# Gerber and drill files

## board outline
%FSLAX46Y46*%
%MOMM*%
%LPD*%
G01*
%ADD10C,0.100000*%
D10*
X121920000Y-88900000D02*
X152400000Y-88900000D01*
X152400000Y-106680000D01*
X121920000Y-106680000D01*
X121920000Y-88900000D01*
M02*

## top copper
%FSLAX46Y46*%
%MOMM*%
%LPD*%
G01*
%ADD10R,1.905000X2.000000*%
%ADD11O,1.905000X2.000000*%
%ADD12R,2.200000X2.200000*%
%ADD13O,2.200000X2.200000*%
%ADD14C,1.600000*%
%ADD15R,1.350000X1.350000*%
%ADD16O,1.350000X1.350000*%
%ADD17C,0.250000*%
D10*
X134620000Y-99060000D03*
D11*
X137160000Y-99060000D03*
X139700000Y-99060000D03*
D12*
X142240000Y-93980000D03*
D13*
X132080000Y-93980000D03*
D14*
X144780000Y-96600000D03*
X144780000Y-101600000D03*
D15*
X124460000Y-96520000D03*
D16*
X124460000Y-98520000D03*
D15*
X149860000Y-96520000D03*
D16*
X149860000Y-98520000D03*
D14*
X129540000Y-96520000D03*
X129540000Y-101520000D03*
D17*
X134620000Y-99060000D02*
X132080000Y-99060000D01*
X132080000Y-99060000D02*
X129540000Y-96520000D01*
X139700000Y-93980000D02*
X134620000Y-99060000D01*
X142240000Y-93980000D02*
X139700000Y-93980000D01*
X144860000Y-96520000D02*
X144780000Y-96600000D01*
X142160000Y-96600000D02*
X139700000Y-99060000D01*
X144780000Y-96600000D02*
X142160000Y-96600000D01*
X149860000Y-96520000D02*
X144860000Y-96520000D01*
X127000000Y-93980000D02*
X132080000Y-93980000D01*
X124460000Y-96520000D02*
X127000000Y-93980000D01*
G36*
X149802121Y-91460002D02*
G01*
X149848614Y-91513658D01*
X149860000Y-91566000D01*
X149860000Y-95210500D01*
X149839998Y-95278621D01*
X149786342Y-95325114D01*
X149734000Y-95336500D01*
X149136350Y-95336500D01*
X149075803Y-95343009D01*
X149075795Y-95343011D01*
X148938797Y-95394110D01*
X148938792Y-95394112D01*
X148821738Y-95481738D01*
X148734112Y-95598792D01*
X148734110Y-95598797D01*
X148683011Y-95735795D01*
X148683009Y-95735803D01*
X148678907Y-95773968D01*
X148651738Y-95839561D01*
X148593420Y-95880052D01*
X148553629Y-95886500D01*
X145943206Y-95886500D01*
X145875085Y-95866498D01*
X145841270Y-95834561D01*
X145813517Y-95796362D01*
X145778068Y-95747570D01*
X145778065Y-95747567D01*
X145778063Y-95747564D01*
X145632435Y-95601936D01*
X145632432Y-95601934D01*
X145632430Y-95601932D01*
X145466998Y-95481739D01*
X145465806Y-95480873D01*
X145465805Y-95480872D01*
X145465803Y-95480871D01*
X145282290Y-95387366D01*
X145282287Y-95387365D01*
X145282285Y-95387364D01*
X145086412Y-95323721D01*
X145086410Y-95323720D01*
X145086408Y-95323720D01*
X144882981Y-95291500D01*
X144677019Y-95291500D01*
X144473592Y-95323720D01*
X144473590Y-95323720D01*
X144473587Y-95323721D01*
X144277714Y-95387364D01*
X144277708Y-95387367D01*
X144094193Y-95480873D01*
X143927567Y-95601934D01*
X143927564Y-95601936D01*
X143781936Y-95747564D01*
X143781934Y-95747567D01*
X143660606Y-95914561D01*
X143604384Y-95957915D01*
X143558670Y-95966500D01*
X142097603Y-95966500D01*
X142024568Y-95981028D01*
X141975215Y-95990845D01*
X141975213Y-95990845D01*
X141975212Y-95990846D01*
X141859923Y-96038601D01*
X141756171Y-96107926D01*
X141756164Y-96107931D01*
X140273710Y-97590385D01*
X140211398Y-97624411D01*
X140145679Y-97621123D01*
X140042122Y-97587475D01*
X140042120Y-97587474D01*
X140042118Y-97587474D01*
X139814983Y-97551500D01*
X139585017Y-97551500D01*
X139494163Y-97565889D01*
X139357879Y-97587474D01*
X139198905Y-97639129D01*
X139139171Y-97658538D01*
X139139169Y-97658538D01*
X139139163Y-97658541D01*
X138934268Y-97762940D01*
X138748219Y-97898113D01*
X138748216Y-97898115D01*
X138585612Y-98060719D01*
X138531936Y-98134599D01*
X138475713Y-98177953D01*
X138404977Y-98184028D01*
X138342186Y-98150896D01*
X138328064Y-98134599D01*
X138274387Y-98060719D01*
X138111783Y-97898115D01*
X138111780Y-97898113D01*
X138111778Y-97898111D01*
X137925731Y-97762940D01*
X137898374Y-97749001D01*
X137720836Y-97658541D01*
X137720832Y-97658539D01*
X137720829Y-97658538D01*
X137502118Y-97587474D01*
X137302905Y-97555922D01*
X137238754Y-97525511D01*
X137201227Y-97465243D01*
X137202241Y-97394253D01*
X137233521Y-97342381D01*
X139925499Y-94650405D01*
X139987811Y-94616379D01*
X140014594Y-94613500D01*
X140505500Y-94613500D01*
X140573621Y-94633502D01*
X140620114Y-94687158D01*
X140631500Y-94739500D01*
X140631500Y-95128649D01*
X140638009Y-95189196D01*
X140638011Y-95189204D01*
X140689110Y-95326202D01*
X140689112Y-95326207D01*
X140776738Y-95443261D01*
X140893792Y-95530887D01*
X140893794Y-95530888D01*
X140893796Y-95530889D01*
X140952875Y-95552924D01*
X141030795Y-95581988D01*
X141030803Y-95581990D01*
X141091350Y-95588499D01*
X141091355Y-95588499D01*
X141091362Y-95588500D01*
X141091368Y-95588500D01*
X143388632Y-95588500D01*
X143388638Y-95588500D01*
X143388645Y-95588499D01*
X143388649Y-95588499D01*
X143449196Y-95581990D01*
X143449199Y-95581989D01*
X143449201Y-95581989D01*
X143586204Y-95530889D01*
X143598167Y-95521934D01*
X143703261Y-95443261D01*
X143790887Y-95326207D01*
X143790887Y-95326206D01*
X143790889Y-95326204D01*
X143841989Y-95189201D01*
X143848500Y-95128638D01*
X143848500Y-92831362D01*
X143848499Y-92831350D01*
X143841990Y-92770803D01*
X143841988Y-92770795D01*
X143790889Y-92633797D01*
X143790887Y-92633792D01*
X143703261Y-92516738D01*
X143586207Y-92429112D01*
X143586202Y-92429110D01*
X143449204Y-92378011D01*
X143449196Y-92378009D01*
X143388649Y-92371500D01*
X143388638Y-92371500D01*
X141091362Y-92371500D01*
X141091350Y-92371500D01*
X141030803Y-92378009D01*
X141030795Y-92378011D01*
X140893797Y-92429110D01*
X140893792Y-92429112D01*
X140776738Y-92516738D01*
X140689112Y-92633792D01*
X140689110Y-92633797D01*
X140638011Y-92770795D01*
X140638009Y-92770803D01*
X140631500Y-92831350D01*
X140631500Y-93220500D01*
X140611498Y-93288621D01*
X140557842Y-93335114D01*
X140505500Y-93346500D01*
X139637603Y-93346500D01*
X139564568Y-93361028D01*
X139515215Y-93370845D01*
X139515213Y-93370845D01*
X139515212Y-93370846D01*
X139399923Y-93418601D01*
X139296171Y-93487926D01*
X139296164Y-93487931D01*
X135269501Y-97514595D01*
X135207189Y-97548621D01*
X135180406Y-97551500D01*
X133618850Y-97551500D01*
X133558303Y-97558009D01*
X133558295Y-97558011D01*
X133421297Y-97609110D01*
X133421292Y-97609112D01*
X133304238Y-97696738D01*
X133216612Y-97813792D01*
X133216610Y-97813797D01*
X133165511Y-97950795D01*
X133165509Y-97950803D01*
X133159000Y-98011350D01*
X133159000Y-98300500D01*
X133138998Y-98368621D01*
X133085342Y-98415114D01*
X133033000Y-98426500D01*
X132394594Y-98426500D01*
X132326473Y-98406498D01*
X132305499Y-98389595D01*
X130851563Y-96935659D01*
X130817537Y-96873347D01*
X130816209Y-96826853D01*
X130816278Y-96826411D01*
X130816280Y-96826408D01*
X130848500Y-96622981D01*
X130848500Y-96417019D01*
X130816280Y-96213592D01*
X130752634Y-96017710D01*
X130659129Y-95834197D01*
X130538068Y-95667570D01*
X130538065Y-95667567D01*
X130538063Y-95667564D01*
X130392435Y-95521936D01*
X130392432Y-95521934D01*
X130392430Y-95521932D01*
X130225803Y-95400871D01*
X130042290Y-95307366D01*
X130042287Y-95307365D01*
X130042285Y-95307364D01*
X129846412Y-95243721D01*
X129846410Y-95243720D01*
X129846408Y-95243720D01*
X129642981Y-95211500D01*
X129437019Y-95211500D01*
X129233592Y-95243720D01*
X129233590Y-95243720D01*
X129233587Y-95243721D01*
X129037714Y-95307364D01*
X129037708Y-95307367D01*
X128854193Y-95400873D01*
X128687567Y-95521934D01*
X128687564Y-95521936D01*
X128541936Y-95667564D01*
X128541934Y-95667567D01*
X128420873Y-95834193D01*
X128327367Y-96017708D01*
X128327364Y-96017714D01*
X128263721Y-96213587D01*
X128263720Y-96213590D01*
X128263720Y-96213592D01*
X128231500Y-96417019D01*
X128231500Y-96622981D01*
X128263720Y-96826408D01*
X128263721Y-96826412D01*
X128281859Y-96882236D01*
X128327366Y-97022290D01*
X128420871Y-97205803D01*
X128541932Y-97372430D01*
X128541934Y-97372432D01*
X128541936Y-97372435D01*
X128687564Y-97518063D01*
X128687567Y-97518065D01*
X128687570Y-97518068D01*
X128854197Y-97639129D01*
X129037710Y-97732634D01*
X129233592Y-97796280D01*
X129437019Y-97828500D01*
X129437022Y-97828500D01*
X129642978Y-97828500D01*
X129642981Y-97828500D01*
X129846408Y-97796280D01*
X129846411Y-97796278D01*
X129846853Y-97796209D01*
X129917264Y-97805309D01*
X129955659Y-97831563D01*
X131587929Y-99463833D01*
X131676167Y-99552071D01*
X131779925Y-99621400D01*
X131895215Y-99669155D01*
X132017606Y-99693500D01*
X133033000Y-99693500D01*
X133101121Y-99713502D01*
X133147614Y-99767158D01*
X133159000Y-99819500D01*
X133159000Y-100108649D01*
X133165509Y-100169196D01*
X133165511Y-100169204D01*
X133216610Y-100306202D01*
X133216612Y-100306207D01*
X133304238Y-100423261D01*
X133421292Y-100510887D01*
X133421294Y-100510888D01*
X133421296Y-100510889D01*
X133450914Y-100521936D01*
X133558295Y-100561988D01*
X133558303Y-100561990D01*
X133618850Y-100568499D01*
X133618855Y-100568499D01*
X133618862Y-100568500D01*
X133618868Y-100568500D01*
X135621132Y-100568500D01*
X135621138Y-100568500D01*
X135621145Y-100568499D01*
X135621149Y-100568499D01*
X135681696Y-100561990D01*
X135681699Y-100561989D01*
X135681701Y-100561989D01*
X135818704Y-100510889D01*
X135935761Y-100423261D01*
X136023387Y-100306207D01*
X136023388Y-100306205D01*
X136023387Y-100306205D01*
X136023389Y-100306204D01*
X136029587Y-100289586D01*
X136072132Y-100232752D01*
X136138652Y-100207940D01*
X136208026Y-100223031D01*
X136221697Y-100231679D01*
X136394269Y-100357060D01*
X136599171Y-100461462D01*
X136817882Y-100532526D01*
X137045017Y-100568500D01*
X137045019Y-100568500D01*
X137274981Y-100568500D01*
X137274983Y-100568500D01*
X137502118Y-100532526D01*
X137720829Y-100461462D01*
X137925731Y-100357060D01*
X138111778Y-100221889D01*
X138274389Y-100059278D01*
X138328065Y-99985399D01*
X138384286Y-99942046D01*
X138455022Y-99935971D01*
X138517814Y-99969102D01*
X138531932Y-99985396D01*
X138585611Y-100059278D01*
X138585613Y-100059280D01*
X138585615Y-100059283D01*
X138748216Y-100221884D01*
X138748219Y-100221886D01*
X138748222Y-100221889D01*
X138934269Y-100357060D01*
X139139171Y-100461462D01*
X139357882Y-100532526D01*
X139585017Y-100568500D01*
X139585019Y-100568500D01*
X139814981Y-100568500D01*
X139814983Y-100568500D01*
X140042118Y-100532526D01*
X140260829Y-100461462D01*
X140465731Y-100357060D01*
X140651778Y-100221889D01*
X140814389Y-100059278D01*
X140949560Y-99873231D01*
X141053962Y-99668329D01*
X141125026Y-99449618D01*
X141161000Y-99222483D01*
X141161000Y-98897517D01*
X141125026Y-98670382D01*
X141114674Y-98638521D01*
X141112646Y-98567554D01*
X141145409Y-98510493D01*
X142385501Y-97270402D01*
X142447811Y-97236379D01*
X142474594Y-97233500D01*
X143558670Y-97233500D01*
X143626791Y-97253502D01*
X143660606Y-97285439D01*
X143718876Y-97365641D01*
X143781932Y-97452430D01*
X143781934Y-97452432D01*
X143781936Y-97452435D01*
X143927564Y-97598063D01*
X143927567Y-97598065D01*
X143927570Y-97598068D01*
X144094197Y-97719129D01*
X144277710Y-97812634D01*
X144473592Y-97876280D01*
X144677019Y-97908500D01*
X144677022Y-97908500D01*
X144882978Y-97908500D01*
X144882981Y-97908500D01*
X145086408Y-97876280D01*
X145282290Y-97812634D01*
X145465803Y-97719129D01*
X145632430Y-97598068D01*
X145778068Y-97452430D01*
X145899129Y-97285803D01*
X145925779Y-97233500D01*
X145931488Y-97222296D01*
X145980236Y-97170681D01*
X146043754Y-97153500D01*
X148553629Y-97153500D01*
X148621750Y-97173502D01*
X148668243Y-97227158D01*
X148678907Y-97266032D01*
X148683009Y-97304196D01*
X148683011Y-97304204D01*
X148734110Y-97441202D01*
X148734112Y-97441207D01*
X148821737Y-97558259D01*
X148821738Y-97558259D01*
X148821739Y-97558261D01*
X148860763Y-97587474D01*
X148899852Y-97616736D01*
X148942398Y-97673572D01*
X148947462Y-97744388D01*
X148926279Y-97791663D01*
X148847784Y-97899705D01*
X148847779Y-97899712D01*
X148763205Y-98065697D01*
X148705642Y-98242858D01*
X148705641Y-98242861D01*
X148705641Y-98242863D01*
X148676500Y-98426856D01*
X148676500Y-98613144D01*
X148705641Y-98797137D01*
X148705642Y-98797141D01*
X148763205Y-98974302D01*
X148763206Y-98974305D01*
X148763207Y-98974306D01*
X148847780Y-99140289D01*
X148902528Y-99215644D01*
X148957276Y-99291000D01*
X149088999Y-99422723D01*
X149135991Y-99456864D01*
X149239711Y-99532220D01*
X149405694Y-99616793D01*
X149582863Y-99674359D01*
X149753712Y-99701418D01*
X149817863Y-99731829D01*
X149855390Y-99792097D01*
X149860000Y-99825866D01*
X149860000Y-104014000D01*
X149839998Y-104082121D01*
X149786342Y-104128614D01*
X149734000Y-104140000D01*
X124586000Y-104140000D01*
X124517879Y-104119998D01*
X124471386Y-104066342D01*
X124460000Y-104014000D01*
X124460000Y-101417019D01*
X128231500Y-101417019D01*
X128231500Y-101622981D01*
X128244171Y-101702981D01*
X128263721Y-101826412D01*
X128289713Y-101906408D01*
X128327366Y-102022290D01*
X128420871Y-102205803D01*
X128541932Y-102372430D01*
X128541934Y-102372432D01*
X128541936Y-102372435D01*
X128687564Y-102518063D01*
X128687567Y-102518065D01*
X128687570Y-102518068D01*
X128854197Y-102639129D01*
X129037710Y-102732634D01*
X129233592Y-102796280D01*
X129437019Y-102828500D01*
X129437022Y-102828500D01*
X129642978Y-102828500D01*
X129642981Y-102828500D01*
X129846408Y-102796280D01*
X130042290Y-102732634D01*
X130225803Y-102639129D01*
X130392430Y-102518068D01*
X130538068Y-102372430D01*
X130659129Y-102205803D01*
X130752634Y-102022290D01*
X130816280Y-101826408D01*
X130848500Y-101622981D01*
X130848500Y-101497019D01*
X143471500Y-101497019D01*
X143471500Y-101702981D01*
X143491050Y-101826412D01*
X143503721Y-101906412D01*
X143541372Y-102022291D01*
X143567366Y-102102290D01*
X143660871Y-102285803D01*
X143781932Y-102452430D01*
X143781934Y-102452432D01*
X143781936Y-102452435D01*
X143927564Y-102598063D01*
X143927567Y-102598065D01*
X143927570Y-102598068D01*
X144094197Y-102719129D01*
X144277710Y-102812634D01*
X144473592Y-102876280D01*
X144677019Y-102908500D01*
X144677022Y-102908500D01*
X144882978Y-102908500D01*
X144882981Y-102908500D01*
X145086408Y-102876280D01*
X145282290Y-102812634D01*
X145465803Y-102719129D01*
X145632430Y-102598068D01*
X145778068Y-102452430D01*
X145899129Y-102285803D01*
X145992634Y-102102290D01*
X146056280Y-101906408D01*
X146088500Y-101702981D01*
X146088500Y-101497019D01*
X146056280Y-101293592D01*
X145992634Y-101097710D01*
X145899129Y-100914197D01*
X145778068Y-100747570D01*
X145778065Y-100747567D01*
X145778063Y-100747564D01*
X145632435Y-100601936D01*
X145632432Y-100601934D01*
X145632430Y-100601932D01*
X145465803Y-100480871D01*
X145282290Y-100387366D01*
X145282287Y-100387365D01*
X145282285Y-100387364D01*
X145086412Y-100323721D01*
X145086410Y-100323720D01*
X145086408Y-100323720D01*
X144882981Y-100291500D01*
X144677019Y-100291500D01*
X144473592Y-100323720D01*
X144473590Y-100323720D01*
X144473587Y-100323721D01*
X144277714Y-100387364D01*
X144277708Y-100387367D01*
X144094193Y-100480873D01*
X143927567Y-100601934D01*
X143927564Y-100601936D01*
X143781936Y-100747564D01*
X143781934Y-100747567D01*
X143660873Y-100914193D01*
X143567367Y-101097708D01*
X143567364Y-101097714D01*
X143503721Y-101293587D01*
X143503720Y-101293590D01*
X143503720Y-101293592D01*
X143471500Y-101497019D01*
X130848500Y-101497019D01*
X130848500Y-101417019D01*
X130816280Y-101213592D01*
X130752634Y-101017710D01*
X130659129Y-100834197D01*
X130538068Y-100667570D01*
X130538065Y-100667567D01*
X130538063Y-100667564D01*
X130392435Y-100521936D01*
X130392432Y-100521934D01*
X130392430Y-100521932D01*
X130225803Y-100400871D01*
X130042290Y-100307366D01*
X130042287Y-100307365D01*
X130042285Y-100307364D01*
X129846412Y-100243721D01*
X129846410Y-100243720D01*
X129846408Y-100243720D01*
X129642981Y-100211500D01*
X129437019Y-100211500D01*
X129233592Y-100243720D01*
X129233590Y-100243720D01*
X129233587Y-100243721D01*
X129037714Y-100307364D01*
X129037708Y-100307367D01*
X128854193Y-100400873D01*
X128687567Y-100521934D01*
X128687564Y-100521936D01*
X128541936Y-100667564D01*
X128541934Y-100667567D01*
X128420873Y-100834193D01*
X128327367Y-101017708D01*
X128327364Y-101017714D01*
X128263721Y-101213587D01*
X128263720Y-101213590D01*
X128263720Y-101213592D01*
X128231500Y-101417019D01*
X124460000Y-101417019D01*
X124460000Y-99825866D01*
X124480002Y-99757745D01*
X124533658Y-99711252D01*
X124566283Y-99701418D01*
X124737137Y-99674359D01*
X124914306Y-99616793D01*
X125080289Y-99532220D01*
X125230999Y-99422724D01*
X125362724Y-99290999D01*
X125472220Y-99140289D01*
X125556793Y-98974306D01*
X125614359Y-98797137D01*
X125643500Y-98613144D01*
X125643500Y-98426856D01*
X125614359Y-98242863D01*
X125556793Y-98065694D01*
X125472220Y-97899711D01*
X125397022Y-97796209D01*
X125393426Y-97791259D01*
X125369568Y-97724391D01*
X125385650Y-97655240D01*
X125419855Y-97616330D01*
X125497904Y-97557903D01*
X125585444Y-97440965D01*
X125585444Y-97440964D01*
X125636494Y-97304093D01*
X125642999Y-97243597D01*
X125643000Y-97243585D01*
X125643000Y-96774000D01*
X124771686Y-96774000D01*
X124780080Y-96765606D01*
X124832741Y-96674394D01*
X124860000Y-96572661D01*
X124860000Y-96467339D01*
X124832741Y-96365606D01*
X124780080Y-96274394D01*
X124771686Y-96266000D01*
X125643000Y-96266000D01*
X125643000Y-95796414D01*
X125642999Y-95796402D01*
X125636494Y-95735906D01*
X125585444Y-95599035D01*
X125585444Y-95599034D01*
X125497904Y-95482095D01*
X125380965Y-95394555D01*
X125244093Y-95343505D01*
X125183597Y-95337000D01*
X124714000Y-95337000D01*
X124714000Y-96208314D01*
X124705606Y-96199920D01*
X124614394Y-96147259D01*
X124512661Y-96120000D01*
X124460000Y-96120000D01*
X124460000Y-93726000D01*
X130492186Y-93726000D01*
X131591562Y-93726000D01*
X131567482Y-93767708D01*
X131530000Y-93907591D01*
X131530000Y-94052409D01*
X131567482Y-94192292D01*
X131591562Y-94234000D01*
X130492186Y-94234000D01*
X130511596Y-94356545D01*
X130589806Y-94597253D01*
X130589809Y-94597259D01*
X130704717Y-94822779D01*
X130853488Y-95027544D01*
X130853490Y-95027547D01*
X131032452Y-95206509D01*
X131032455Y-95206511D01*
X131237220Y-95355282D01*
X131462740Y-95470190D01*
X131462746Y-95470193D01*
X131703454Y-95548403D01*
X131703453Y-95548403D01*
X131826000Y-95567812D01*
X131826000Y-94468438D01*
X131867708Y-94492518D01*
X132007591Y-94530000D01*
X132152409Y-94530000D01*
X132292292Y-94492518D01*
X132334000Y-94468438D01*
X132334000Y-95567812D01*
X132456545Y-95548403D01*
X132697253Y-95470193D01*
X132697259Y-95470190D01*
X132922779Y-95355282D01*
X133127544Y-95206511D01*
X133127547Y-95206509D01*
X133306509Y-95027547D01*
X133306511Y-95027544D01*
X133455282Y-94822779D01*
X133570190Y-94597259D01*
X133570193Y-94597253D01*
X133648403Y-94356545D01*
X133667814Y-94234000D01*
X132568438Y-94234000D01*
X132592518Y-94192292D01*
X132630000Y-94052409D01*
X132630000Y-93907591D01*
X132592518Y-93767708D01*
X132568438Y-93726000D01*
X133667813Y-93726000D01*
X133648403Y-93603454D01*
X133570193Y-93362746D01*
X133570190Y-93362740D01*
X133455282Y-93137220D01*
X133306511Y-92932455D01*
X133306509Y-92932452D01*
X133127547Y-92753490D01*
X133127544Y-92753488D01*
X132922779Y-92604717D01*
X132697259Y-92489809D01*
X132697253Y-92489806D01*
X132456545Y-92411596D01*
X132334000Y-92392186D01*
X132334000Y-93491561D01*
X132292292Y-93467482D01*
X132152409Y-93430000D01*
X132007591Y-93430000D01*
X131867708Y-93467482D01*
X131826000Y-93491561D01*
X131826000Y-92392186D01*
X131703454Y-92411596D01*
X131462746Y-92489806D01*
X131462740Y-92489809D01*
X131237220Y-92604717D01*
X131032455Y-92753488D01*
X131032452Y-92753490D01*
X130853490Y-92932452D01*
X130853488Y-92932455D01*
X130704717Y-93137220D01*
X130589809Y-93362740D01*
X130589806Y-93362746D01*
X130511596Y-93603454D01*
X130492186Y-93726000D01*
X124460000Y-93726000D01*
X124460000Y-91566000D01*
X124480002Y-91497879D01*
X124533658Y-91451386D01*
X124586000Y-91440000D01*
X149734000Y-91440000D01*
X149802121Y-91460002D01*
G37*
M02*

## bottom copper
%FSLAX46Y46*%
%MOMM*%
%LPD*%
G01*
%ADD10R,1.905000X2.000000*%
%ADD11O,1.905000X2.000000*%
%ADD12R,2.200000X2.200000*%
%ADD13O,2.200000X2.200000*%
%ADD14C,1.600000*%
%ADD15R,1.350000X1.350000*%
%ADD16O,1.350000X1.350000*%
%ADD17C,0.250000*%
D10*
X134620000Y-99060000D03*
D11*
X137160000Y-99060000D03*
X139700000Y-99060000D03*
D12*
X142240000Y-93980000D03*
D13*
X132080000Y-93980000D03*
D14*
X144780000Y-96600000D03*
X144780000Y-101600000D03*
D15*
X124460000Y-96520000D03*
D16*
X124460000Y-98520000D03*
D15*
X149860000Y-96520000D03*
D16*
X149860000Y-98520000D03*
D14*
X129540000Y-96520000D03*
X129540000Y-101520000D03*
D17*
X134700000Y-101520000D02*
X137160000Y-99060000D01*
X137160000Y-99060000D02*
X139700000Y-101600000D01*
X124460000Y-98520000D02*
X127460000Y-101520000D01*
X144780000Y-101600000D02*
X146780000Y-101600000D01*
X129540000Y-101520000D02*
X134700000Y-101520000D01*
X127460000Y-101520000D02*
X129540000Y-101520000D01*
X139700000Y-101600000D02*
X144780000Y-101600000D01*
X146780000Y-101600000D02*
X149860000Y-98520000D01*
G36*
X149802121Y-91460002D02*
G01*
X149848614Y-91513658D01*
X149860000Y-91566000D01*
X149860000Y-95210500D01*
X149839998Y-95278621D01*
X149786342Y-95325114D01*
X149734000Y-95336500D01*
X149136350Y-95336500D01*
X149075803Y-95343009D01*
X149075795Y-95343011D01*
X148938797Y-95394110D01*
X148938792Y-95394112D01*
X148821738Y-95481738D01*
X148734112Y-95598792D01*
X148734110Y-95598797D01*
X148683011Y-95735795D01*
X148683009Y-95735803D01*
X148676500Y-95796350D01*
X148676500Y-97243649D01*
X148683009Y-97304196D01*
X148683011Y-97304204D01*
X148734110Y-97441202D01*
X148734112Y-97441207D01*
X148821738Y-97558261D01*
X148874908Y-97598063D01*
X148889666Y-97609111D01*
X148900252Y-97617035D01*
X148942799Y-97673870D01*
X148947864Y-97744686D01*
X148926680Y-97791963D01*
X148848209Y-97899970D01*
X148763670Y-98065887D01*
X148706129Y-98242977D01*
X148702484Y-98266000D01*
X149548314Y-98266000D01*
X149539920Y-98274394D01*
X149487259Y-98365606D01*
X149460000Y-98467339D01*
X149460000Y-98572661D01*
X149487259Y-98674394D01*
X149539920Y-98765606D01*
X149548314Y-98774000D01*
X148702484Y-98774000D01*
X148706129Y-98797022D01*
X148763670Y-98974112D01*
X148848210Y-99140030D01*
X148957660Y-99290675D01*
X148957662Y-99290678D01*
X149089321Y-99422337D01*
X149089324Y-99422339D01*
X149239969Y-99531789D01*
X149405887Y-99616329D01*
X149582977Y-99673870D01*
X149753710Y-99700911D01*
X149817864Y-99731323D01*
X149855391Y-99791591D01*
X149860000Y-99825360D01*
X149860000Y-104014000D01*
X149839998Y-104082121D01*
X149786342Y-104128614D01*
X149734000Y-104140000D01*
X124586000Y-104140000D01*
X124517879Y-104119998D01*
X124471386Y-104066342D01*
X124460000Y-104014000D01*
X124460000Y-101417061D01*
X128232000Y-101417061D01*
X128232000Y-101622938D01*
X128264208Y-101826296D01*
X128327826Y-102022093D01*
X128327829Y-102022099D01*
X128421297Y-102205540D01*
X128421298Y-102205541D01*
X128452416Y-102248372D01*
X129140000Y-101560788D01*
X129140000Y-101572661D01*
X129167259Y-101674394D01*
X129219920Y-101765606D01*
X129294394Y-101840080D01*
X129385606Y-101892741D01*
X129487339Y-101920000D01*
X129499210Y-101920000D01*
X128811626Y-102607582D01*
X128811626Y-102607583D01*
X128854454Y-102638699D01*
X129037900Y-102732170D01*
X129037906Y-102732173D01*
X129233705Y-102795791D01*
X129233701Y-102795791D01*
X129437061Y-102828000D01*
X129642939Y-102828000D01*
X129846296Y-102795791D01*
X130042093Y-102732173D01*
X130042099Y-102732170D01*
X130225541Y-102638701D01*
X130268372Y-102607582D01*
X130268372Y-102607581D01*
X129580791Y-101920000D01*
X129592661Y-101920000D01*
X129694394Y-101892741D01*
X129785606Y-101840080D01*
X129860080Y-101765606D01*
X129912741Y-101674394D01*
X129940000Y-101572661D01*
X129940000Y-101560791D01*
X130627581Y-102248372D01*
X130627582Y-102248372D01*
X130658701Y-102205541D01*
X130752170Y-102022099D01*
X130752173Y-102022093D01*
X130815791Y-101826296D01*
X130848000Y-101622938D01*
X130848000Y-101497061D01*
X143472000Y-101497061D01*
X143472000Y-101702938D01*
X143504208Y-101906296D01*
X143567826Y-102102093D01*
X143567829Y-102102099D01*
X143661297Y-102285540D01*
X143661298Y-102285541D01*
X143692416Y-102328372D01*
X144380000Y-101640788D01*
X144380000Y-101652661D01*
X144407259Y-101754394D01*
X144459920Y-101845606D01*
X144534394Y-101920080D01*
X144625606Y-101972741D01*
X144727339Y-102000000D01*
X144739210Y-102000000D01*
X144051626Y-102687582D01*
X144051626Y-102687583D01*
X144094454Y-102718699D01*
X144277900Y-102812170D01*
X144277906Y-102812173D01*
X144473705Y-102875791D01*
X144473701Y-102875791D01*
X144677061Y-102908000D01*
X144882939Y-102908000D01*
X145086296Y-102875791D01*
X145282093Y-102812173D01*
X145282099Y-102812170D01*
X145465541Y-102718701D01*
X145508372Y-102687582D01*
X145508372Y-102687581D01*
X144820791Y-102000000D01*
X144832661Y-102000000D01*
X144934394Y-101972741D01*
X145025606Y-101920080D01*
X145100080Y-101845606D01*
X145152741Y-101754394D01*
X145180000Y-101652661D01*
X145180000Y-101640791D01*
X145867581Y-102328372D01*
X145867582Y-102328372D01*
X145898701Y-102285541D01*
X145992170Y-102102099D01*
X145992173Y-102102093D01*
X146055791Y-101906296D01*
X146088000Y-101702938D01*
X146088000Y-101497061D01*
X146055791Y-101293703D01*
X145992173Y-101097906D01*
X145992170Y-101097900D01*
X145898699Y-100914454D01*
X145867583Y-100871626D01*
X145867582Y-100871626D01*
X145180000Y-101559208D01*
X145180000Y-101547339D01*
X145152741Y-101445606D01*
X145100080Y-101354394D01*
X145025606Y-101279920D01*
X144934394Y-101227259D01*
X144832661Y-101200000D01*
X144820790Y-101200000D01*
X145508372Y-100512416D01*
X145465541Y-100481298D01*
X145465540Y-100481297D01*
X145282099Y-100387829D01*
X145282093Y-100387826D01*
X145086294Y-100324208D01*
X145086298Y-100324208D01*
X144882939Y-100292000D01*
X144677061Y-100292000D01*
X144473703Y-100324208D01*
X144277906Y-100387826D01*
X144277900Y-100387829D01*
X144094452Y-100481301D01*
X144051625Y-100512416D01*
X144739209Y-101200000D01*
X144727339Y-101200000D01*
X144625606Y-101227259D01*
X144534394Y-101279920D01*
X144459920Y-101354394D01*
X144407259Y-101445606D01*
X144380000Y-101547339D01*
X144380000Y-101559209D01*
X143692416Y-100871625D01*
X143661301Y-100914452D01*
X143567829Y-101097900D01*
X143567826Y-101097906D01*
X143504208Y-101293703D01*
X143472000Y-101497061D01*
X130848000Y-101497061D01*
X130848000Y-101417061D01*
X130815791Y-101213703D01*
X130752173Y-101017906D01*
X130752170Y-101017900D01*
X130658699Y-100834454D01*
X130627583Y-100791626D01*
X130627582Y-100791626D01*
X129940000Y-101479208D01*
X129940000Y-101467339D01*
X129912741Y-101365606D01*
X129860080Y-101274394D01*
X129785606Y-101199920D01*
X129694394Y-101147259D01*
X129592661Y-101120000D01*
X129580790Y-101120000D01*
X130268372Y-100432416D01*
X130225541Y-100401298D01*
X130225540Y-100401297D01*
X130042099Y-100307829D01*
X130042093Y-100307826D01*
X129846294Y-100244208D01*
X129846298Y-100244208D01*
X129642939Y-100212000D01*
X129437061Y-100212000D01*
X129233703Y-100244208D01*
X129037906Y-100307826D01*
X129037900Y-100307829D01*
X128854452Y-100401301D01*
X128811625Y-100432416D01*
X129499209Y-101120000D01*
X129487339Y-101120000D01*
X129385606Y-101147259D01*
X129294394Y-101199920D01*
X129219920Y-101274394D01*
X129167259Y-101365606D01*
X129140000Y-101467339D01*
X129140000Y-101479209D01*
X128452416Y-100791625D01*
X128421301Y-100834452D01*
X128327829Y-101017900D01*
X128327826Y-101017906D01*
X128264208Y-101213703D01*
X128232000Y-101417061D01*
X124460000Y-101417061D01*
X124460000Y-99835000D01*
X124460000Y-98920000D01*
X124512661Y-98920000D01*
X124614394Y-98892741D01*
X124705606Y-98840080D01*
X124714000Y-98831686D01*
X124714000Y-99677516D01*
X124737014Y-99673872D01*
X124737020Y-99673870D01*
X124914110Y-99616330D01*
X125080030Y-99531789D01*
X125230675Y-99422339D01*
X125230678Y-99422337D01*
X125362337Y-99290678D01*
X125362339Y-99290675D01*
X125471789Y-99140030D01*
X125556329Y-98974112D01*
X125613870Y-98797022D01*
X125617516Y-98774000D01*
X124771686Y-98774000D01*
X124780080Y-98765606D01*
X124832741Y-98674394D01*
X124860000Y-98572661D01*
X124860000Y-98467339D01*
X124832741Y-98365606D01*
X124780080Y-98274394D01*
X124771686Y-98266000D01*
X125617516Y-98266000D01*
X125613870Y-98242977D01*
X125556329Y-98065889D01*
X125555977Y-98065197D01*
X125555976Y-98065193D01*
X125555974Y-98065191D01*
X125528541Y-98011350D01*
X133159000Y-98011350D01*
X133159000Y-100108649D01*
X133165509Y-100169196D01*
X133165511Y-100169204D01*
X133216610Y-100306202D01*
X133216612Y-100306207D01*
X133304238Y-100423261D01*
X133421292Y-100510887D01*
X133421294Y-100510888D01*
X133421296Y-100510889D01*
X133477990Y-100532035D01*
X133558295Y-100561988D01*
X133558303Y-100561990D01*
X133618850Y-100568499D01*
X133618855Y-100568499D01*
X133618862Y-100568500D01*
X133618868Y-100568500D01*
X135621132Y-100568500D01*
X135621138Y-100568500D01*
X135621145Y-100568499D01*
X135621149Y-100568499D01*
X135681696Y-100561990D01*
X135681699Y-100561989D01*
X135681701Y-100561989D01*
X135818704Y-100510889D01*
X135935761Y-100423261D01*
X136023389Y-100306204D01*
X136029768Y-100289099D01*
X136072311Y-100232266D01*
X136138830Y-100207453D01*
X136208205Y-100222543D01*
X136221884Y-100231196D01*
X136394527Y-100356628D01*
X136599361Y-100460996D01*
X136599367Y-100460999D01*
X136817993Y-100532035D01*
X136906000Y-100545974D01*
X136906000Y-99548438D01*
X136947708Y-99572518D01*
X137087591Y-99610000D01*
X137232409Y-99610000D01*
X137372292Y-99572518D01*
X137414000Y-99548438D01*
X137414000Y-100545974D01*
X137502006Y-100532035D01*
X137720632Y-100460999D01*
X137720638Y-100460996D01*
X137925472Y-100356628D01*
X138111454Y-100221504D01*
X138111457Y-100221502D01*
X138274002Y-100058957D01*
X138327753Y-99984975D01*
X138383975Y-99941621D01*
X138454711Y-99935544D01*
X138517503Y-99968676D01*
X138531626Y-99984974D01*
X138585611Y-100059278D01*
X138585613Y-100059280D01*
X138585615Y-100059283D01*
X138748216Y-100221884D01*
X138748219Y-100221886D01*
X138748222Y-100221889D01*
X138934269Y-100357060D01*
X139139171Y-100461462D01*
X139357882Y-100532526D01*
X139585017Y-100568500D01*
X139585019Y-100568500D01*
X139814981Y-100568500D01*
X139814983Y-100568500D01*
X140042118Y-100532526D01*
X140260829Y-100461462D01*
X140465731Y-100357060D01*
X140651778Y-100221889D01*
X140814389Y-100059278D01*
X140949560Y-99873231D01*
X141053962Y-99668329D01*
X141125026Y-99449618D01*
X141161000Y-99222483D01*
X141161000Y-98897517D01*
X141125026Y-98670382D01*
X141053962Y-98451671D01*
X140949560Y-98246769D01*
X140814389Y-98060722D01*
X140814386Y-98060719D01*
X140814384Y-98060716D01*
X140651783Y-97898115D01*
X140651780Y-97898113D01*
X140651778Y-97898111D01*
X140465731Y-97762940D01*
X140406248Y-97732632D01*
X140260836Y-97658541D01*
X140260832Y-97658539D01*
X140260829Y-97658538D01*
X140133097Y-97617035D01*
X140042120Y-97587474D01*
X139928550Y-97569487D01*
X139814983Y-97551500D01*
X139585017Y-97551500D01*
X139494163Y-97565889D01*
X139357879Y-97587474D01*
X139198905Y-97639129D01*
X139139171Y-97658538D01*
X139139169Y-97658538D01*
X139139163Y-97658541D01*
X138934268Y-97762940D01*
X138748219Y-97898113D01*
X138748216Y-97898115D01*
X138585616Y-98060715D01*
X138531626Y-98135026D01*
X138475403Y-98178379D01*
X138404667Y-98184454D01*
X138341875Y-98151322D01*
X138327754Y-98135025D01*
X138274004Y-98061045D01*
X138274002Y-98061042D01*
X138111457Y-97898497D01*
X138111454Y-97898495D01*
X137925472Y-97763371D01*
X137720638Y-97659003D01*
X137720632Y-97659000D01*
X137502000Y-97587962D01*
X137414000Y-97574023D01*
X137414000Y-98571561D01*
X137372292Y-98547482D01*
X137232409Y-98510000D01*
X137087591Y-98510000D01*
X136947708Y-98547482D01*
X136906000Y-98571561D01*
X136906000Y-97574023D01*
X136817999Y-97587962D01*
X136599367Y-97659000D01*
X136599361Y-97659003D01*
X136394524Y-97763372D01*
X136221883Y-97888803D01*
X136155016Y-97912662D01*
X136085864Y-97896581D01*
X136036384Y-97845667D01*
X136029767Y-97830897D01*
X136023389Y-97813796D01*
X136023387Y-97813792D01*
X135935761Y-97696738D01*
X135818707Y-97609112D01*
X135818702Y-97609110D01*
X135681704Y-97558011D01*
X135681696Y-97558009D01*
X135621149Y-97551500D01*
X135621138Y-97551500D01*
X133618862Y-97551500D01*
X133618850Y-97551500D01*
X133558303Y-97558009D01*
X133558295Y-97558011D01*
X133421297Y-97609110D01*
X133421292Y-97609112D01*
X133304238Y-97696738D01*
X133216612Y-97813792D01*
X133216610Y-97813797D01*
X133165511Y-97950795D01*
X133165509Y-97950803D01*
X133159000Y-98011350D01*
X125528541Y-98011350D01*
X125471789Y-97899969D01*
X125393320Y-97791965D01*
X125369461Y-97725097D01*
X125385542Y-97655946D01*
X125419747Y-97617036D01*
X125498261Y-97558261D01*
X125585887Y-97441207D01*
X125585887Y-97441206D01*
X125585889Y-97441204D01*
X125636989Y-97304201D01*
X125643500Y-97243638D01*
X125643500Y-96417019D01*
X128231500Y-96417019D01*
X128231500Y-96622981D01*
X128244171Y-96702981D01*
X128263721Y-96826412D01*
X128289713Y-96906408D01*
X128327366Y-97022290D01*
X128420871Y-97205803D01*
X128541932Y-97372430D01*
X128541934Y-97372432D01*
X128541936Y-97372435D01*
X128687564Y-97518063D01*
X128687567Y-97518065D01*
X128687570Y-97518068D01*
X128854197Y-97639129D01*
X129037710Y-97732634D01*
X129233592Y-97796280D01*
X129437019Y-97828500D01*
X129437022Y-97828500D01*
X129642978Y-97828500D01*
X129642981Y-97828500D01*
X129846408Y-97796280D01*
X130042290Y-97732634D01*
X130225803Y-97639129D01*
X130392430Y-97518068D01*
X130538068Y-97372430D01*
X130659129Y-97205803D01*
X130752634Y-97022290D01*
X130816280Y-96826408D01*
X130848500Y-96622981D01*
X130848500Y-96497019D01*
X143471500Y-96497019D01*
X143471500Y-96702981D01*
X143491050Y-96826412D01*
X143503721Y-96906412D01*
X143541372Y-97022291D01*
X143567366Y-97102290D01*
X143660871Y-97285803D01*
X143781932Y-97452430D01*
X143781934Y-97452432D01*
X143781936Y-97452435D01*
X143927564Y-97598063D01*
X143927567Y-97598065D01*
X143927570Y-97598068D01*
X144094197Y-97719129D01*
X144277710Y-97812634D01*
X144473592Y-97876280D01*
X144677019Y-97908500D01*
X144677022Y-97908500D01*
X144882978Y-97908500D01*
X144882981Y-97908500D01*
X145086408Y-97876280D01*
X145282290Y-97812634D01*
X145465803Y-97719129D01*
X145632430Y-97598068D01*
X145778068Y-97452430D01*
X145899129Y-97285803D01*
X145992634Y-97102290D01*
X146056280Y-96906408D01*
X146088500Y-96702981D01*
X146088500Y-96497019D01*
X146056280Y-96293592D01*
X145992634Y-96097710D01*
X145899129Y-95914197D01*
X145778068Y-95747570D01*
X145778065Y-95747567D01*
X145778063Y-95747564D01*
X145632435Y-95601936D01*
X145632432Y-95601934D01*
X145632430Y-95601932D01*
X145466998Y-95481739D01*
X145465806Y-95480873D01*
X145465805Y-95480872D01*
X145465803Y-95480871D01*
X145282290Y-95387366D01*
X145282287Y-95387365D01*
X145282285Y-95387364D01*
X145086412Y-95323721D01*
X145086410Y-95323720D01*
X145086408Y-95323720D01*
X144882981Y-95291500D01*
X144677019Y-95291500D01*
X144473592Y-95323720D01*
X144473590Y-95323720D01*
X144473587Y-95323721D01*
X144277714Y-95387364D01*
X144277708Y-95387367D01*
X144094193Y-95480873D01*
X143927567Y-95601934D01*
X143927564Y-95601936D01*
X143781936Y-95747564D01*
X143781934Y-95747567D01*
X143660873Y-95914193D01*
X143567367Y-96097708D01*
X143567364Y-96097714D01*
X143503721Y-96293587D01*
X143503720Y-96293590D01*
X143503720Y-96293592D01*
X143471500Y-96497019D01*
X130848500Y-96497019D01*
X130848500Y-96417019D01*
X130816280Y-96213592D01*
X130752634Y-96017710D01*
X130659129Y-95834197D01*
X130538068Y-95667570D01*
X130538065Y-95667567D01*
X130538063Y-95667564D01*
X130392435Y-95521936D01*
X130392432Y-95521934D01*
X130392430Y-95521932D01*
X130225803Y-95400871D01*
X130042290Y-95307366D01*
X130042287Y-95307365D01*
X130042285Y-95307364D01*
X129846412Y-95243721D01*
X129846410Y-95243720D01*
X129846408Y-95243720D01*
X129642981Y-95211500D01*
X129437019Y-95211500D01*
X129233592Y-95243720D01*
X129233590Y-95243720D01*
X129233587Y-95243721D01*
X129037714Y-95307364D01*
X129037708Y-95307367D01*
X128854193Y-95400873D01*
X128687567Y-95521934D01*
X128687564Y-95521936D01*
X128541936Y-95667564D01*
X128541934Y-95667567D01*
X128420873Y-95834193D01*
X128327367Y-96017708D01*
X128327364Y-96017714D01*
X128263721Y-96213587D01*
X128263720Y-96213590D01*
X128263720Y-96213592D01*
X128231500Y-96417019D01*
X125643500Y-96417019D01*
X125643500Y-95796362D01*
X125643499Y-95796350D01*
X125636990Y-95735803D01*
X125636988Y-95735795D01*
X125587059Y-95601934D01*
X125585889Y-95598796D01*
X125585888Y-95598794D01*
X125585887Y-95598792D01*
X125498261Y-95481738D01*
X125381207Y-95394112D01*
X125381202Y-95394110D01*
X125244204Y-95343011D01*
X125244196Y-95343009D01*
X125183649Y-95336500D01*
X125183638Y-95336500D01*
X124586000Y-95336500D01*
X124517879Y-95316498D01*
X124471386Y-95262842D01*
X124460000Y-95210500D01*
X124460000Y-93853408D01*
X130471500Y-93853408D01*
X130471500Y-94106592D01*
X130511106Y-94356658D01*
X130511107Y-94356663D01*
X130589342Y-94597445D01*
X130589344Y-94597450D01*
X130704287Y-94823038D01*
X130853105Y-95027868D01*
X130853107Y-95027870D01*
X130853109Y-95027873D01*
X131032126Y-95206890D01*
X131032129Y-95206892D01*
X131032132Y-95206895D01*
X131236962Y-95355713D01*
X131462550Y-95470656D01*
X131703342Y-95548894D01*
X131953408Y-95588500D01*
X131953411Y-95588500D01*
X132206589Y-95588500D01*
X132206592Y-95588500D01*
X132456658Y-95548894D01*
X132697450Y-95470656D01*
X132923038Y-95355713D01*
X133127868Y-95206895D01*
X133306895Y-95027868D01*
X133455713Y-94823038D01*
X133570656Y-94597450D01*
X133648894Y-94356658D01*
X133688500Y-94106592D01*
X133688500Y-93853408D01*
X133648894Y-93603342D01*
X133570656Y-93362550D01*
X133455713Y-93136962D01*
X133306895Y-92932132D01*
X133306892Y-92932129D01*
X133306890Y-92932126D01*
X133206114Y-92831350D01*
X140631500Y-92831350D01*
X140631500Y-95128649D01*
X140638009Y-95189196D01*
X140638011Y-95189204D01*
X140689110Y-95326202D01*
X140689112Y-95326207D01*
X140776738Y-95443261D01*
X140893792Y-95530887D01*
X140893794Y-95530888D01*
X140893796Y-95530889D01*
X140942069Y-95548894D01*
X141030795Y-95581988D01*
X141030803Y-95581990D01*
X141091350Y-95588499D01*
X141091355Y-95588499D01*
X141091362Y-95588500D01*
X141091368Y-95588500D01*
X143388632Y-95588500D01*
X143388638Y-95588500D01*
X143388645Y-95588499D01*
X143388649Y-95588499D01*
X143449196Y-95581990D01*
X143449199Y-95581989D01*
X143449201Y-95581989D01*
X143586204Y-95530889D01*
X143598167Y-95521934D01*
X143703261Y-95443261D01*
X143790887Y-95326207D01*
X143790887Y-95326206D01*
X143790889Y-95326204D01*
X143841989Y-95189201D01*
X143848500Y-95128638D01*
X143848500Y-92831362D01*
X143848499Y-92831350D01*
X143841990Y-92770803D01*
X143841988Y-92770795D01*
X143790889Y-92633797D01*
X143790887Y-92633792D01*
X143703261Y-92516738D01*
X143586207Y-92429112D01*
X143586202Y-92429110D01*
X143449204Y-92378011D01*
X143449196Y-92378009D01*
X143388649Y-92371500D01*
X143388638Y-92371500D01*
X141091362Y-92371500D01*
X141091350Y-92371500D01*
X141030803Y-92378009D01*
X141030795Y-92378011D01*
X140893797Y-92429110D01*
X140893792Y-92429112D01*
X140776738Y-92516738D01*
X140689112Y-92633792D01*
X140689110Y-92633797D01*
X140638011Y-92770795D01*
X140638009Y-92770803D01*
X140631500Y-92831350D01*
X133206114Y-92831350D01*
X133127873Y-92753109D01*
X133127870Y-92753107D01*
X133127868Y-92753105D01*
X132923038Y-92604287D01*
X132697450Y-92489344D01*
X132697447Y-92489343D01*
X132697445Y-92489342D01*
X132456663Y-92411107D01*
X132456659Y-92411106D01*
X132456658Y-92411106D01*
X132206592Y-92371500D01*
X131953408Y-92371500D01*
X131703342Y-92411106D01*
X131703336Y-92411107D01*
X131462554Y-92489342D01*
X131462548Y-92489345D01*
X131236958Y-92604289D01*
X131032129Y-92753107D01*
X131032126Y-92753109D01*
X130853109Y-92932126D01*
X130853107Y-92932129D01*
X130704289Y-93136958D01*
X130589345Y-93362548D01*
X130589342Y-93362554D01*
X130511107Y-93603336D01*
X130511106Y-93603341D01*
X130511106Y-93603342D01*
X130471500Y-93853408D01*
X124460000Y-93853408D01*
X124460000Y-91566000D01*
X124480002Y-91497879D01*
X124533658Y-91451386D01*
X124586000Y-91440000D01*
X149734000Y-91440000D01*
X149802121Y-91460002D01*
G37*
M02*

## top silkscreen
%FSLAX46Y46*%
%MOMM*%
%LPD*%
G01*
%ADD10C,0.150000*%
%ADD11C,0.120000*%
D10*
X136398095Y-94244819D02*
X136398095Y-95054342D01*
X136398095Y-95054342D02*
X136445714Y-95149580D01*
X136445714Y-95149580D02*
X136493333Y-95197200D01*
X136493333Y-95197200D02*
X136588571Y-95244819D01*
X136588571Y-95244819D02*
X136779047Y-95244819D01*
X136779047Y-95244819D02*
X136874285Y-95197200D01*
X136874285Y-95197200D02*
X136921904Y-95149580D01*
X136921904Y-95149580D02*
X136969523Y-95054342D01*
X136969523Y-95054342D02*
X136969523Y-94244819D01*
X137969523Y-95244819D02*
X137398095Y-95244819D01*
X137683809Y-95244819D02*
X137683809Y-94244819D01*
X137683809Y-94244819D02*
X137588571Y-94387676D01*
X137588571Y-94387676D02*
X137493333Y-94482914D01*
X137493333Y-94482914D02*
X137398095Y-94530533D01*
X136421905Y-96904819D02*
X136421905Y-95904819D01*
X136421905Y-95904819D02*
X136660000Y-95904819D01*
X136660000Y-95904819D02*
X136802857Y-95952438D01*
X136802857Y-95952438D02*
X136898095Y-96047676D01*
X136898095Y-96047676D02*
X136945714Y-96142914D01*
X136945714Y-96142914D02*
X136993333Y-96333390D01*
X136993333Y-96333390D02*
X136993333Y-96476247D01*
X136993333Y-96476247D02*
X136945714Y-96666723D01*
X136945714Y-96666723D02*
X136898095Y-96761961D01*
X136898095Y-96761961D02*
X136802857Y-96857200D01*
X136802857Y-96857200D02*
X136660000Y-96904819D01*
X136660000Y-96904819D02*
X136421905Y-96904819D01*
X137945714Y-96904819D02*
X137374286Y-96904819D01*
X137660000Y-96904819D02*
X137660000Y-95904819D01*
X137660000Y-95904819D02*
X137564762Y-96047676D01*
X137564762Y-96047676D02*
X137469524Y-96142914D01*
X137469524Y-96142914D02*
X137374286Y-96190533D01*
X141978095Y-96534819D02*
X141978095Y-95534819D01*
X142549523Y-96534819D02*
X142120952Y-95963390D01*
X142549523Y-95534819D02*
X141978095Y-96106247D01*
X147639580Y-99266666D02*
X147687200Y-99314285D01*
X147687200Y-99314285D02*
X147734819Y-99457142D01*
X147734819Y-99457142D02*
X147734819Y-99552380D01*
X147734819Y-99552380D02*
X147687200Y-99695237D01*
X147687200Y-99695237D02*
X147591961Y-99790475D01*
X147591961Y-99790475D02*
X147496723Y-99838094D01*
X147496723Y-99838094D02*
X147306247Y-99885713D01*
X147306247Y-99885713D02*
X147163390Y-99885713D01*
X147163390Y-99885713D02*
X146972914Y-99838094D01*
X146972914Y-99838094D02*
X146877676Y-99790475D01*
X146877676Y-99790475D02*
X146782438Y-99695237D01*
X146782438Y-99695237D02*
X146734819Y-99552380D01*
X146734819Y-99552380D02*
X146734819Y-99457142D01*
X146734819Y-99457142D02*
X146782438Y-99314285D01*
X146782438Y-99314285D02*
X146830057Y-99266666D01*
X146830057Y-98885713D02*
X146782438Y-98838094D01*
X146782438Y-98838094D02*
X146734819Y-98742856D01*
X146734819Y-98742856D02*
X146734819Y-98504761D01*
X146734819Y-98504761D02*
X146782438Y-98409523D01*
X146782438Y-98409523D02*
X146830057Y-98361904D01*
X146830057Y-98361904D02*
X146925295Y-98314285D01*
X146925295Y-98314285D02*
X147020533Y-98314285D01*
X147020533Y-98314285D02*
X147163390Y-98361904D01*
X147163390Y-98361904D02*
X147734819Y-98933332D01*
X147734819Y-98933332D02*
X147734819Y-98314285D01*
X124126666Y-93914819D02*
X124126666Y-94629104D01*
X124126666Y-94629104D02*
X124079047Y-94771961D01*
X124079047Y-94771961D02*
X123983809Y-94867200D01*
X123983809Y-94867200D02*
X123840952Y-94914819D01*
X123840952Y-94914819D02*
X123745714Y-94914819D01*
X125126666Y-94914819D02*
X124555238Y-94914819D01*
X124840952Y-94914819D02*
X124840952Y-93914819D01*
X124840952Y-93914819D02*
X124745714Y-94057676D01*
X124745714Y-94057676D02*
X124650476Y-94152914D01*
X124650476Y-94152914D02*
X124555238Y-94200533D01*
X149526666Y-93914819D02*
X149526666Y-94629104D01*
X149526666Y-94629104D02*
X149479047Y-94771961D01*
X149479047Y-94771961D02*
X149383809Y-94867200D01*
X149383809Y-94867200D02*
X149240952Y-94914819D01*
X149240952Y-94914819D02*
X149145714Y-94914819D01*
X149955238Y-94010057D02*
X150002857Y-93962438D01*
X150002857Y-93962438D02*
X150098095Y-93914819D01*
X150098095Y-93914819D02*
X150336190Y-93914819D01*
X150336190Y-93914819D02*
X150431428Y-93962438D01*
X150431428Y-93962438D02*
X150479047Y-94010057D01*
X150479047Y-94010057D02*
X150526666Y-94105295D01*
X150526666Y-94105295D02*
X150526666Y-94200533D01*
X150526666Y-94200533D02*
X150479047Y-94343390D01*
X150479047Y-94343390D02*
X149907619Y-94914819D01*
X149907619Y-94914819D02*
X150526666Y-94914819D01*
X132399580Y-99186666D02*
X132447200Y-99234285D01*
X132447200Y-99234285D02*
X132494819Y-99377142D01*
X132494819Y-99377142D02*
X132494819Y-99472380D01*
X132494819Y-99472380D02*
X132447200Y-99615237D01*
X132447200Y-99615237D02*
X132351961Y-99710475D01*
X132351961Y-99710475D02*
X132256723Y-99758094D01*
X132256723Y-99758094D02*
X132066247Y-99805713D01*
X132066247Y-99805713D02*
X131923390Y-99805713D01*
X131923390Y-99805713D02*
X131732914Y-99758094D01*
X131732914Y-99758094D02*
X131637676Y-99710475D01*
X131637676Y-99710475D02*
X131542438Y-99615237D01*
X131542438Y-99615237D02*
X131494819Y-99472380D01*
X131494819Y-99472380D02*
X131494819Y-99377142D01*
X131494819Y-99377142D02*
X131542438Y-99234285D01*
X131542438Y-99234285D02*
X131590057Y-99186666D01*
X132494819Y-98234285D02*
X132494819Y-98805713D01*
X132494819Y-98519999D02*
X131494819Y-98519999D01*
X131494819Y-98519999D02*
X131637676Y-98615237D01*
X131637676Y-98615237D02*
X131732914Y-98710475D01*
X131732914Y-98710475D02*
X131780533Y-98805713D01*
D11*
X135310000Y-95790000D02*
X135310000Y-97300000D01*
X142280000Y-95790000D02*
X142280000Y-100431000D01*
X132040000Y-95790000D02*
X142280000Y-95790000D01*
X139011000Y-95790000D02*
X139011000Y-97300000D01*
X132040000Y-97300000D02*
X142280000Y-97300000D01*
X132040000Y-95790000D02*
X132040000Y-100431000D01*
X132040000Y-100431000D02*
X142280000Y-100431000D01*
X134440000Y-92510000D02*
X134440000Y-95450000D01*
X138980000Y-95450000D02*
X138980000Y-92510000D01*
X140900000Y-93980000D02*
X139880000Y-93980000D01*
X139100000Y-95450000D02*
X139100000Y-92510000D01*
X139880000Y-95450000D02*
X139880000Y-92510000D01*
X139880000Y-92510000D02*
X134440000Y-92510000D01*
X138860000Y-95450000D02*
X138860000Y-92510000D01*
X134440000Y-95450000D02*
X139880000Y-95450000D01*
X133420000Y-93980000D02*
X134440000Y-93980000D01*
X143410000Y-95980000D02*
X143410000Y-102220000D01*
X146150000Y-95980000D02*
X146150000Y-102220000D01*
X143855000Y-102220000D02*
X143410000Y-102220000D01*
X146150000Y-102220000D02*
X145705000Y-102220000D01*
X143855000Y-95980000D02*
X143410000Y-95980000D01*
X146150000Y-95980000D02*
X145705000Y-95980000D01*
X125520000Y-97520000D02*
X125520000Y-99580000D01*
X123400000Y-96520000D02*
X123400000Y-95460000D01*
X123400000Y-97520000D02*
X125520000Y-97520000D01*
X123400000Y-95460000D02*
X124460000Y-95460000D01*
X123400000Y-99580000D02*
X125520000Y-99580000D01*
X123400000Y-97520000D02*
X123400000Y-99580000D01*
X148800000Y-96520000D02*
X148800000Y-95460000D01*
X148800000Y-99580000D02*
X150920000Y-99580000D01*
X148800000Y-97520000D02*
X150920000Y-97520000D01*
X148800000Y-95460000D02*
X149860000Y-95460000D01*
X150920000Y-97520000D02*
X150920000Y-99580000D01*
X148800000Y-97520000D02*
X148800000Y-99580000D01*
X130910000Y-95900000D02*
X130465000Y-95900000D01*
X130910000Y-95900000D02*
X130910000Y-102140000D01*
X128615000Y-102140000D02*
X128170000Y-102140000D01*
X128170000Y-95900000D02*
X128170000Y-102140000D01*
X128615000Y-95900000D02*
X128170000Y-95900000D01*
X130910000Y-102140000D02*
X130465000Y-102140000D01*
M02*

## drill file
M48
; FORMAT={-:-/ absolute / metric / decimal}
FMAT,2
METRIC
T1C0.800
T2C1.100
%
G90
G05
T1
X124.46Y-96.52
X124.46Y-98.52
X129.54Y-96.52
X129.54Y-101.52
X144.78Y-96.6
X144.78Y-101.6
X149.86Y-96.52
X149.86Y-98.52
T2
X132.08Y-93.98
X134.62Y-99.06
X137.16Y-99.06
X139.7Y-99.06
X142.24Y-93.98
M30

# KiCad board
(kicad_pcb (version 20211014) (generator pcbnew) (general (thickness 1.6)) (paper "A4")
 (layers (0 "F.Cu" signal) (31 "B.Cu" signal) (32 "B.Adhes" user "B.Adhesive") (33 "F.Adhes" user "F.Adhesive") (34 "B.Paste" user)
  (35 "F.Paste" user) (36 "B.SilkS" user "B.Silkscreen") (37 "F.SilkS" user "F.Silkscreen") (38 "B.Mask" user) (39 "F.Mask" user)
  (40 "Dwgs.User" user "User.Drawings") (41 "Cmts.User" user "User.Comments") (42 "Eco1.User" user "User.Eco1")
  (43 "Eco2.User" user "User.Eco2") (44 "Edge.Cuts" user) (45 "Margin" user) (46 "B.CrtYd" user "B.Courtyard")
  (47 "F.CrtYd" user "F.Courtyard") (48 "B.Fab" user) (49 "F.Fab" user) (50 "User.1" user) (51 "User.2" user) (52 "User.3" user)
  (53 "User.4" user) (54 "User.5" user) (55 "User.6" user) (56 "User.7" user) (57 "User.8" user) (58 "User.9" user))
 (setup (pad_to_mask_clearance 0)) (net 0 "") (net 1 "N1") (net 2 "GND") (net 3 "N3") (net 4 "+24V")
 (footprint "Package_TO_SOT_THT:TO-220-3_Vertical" (layer "F.Cu") (at 134.62 99.06)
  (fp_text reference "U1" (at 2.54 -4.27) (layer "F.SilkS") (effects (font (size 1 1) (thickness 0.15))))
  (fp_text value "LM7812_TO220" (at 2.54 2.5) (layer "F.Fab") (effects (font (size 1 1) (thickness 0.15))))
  (fp_line (start 0.69 -3.27) (end 0.69 -1.76) (layer "F.SilkS") (width 0.12))
  (fp_line (start 7.66 -3.27) (end 7.66 1.371) (layer "F.SilkS") (width 0.12))
  (fp_line (start -2.58 -3.27) (end 7.66 -3.27) (layer "F.SilkS") (width 0.12))
  (fp_line (start 4.391 -3.27) (end 4.391 -1.76) (layer "F.SilkS") (width 0.12))
  (fp_line (start -2.58 -1.76) (end 7.66 -1.76) (layer "F.SilkS") (width 0.12))
  (fp_line (start -2.58 -3.27) (end -2.58 1.371) (layer "F.SilkS") (width 0.12))
  (fp_line (start -2.58 1.371) (end 7.66 1.371) (layer "F.SilkS") (width 0.12))
  (pad "1" thru_hole rect (at 0 0) (size 1.905 2) (drill 1.1) (layers *.Cu *.Mask) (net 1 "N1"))
  (pad "2" thru_hole oval (at 2.54 0) (size 1.905 2) (drill 1.1) (layers *.Cu *.Mask) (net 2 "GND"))
  (pad "3" thru_hole oval (at 5.08 0) (size 1.905 2) (drill 1.1) (layers *.Cu *.Mask) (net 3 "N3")))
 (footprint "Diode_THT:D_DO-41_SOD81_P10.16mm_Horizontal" (layer "F.Cu") (at 142.24 93.98 180)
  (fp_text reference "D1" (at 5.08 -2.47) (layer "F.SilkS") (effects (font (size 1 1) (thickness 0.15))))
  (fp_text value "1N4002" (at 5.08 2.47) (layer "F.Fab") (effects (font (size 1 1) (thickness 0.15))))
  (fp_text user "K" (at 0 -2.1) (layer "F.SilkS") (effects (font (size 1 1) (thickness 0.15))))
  (fp_line (start 7.8 1.47) (end 7.8 -1.47) (layer "F.SilkS") (width 0.12))
  (fp_line (start 3.26 -1.47) (end 3.26 1.47) (layer "F.SilkS") (width 0.12))
  (fp_line (start 1.34 0) (end 2.36 0) (layer "F.SilkS") (width 0.12))
  (fp_line (start 3.14 -1.47) (end 3.14 1.47) (layer "F.SilkS") (width 0.12))
  (fp_line (start 2.36 -1.47) (end 2.36 1.47) (layer "F.SilkS") (width 0.12))
  (fp_line (start 2.36 1.47) (end 7.8 1.47) (layer "F.SilkS") (width 0.12))
  (fp_line (start 3.38 -1.47) (end 3.38 1.47) (layer "F.SilkS") (width 0.12))
  (fp_line (start 7.8 -1.47) (end 2.36 -1.47) (layer "F.SilkS") (width 0.12))
  (fp_line (start 8.82 0) (end 7.8 0) (layer "F.SilkS") (width 0.12))
  (pad "1" thru_hole rect (at 0 0 180) (size 2.2 2.2) (drill 1.1) (layers *.Cu *.Mask) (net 1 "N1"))
  (pad "2" thru_hole oval (at 10.16 0 180) (size 2.2 2.2) (drill 1.1) (layers *.Cu *.Mask) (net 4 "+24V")))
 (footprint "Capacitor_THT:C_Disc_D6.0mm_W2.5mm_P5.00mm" (layer "F.Cu") (at 144.78 96.6 -90)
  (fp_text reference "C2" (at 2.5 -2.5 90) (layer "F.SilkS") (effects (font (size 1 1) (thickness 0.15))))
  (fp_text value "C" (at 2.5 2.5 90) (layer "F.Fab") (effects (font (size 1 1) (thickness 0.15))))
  (fp_line (start -0.62 1.37) (end 5.62 1.37) (layer "F.SilkS") (width 0.12))
  (fp_line (start -0.62 -1.37) (end 5.62 -1.37) (layer "F.SilkS") (width 0.12))
  (fp_line (start 5.62 0.925) (end 5.62 1.37) (layer "F.SilkS") (width 0.12))
  (fp_line (start 5.62 -1.37) (end 5.62 -0.925) (layer "F.SilkS") (width 0.12))
  (fp_line (start -0.62 0.925) (end -0.62 1.37) (layer "F.SilkS") (width 0.12))
  (fp_line (start -0.62 -1.37) (end -0.62 -0.925) (layer "F.SilkS") (width 0.12))
  (pad "1" thru_hole circle (at 0 0 270) (size 1.6 1.6) (drill 0.8) (layers *.Cu *.Mask) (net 3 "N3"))
  (pad "2" thru_hole circle (at 5 0 270) (size 1.6 1.6) (drill 0.8) (layers *.Cu *.Mask) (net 2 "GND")))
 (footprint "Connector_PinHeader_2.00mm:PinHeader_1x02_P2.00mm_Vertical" (layer "F.Cu") (at 124.46 96.52)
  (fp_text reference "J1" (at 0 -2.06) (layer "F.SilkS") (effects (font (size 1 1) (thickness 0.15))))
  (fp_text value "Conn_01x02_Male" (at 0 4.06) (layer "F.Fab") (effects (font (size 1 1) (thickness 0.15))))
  (fp_line (start 1.06 1) (end 1.06 3.06) (layer "F.SilkS") (width 0.12))
  (fp_line (start -1.06 0) (end -1.06 -1.06) (layer "F.SilkS") (width 0.12))
  (fp_line (start -1.06 1) (end 1.06 1) (layer "F.SilkS") (width 0.12))
  (fp_line (start -1.06 -1.06) (end 0 -1.06) (layer "F.SilkS") (width 0.12))
  (fp_line (start -1.06 3.06) (end 1.06 3.06) (layer "F.SilkS") (width 0.12))
  (fp_line (start -1.06 1) (end -1.06 3.06) (layer "F.SilkS") (width 0.12))
  (pad "1" thru_hole rect (at 0 0) (size 1.35 1.35) (drill 0.8) (layers *.Cu *.Mask) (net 4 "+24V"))
  (pad "2" thru_hole oval (at 0 2) (size 1.35 1.35) (drill 0.8) (layers *.Cu *.Mask) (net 2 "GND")))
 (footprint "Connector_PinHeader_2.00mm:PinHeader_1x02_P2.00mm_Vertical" (layer "F.Cu") (at 149.86 96.52)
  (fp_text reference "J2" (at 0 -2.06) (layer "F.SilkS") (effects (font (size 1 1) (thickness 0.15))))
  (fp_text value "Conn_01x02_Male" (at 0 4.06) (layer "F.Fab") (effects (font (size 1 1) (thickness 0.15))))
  (fp_line (start -1.06 0) (end -1.06 -1.06) (layer "F.SilkS") (width 0.12))
  (fp_line (start -1.06 3.06) (end 1.06 3.06) (layer "F.SilkS") (width 0.12))
  (fp_line (start -1.06 1) (end 1.06 1) (layer "F.SilkS") (width 0.12))
  (fp_line (start -1.06 -1.06) (end 0 -1.06) (layer "F.SilkS") (width 0.12))
  (fp_line (start 1.06 1) (end 1.06 3.06) (layer "F.SilkS") (width 0.12))
  (fp_line (start -1.06 1) (end -1.06 3.06) (layer "F.SilkS") (width 0.12))
  (pad "1" thru_hole rect (at 0 0) (size 1.35 1.35) (drill 0.8) (layers *.Cu *.Mask) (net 3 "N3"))
  (pad "2" thru_hole oval (at 0 2) (size 1.35 1.35) (drill 0.8) (layers *.Cu *.Mask) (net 2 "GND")))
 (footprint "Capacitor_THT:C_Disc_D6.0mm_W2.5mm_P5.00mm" (layer "F.Cu") (at 129.54 96.52 -90)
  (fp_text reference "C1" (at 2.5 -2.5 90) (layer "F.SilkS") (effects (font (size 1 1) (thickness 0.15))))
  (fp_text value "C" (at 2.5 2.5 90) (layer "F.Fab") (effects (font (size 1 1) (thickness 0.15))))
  (fp_line (start -0.62 -1.37) (end -0.62 -0.925) (layer "F.SilkS") (width 0.12))
  (fp_line (start -0.62 -1.37) (end 5.62 -1.37) (layer "F.SilkS") (width 0.12))
  (fp_line (start 5.62 0.925) (end 5.62 1.37) (layer "F.SilkS") (width 0.12))
  (fp_line (start -0.62 1.37) (end 5.62 1.37) (layer "F.SilkS") (width 0.12))
  (fp_line (start -0.62 0.925) (end -0.62 1.37) (layer "F.SilkS") (width 0.12))
  (fp_line (start 5.62 -1.37) (end 5.62 -0.925) (layer "F.SilkS") (width 0.12))
  (pad "1" thru_hole circle (at 0 0 270) (size 1.6 1.6) (drill 0.8) (layers *.Cu *.Mask) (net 1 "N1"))
  (pad "2" thru_hole circle (at 5 0 270) (size 1.6 1.6) (drill 0.8) (layers *.Cu *.Mask) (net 2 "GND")))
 (gr_rect (start 121.92 88.9) (end 152.4 106.68) (layer "Edge.Cuts") (width 0.1) (fill none))
 (segment (start 134.62 99.06) (end 132.08 99.06) (width 0.25) (layer "F.Cu") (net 1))
 (segment (start 132.08 99.06) (end 129.54 96.52) (width 0.25) (layer "F.Cu") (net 1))
 (segment (start 139.7 93.98) (end 134.62 99.06) (width 0.25) (layer "F.Cu") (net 1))
 (segment (start 142.24 93.98) (end 139.7 93.98) (width 0.25) (layer "F.Cu") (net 1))
 (segment (start 134.7 101.52) (end 137.16 99.06) (width 0.25) (layer "B.Cu") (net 2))
 (segment (start 137.16 99.06) (end 139.7 101.6) (width 0.25) (layer "B.Cu") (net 2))
 (segment (start 124.46 98.52) (end 127.46 101.52) (width 0.25) (layer "B.Cu") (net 2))
 (segment (start 144.78 101.6) (end 146.78 101.6) (width 0.25) (layer "B.Cu") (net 2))
 (segment (start 129.54 101.52) (end 134.7 101.52) (width 0.25) (layer "B.Cu") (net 2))
 (segment (start 127.46 101.52) (end 129.54 101.52) (width 0.25) (layer "B.Cu") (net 2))
 (segment (start 139.7 101.6) (end 144.78 101.6) (width 0.25) (layer "B.Cu") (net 2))
 (segment (start 146.78 101.6) (end 149.86 98.52) (width 0.25) (layer "B.Cu") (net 2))
 (segment (start 144.86 96.52) (end 144.78 96.6) (width 0.25) (layer "F.Cu") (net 3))
 (segment (start 142.16 96.6) (end 139.7 99.06) (width 0.25) (layer "F.Cu") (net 3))
 (segment (start 144.78 96.6) (end 142.16 96.6) (width 0.25) (layer "F.Cu") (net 3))
 (segment (start 149.86 96.52) (end 144.86 96.52) (width 0.25) (layer "F.Cu") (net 3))
 (segment (start 127 93.98) (end 132.08 93.98) (width 0.25) (layer "F.Cu") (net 4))
 (segment (start 124.46 96.52) (end 127 93.98) (width 0.25) (layer "F.Cu") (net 4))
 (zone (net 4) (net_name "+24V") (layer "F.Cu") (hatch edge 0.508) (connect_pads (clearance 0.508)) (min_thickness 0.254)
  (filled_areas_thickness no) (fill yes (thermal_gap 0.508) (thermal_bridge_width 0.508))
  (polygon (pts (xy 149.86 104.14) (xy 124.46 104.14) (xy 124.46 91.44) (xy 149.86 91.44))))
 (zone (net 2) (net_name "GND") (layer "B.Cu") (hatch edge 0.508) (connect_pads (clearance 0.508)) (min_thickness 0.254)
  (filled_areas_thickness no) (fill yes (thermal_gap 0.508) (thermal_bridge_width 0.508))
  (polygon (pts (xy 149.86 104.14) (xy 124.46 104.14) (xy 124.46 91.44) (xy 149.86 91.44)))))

